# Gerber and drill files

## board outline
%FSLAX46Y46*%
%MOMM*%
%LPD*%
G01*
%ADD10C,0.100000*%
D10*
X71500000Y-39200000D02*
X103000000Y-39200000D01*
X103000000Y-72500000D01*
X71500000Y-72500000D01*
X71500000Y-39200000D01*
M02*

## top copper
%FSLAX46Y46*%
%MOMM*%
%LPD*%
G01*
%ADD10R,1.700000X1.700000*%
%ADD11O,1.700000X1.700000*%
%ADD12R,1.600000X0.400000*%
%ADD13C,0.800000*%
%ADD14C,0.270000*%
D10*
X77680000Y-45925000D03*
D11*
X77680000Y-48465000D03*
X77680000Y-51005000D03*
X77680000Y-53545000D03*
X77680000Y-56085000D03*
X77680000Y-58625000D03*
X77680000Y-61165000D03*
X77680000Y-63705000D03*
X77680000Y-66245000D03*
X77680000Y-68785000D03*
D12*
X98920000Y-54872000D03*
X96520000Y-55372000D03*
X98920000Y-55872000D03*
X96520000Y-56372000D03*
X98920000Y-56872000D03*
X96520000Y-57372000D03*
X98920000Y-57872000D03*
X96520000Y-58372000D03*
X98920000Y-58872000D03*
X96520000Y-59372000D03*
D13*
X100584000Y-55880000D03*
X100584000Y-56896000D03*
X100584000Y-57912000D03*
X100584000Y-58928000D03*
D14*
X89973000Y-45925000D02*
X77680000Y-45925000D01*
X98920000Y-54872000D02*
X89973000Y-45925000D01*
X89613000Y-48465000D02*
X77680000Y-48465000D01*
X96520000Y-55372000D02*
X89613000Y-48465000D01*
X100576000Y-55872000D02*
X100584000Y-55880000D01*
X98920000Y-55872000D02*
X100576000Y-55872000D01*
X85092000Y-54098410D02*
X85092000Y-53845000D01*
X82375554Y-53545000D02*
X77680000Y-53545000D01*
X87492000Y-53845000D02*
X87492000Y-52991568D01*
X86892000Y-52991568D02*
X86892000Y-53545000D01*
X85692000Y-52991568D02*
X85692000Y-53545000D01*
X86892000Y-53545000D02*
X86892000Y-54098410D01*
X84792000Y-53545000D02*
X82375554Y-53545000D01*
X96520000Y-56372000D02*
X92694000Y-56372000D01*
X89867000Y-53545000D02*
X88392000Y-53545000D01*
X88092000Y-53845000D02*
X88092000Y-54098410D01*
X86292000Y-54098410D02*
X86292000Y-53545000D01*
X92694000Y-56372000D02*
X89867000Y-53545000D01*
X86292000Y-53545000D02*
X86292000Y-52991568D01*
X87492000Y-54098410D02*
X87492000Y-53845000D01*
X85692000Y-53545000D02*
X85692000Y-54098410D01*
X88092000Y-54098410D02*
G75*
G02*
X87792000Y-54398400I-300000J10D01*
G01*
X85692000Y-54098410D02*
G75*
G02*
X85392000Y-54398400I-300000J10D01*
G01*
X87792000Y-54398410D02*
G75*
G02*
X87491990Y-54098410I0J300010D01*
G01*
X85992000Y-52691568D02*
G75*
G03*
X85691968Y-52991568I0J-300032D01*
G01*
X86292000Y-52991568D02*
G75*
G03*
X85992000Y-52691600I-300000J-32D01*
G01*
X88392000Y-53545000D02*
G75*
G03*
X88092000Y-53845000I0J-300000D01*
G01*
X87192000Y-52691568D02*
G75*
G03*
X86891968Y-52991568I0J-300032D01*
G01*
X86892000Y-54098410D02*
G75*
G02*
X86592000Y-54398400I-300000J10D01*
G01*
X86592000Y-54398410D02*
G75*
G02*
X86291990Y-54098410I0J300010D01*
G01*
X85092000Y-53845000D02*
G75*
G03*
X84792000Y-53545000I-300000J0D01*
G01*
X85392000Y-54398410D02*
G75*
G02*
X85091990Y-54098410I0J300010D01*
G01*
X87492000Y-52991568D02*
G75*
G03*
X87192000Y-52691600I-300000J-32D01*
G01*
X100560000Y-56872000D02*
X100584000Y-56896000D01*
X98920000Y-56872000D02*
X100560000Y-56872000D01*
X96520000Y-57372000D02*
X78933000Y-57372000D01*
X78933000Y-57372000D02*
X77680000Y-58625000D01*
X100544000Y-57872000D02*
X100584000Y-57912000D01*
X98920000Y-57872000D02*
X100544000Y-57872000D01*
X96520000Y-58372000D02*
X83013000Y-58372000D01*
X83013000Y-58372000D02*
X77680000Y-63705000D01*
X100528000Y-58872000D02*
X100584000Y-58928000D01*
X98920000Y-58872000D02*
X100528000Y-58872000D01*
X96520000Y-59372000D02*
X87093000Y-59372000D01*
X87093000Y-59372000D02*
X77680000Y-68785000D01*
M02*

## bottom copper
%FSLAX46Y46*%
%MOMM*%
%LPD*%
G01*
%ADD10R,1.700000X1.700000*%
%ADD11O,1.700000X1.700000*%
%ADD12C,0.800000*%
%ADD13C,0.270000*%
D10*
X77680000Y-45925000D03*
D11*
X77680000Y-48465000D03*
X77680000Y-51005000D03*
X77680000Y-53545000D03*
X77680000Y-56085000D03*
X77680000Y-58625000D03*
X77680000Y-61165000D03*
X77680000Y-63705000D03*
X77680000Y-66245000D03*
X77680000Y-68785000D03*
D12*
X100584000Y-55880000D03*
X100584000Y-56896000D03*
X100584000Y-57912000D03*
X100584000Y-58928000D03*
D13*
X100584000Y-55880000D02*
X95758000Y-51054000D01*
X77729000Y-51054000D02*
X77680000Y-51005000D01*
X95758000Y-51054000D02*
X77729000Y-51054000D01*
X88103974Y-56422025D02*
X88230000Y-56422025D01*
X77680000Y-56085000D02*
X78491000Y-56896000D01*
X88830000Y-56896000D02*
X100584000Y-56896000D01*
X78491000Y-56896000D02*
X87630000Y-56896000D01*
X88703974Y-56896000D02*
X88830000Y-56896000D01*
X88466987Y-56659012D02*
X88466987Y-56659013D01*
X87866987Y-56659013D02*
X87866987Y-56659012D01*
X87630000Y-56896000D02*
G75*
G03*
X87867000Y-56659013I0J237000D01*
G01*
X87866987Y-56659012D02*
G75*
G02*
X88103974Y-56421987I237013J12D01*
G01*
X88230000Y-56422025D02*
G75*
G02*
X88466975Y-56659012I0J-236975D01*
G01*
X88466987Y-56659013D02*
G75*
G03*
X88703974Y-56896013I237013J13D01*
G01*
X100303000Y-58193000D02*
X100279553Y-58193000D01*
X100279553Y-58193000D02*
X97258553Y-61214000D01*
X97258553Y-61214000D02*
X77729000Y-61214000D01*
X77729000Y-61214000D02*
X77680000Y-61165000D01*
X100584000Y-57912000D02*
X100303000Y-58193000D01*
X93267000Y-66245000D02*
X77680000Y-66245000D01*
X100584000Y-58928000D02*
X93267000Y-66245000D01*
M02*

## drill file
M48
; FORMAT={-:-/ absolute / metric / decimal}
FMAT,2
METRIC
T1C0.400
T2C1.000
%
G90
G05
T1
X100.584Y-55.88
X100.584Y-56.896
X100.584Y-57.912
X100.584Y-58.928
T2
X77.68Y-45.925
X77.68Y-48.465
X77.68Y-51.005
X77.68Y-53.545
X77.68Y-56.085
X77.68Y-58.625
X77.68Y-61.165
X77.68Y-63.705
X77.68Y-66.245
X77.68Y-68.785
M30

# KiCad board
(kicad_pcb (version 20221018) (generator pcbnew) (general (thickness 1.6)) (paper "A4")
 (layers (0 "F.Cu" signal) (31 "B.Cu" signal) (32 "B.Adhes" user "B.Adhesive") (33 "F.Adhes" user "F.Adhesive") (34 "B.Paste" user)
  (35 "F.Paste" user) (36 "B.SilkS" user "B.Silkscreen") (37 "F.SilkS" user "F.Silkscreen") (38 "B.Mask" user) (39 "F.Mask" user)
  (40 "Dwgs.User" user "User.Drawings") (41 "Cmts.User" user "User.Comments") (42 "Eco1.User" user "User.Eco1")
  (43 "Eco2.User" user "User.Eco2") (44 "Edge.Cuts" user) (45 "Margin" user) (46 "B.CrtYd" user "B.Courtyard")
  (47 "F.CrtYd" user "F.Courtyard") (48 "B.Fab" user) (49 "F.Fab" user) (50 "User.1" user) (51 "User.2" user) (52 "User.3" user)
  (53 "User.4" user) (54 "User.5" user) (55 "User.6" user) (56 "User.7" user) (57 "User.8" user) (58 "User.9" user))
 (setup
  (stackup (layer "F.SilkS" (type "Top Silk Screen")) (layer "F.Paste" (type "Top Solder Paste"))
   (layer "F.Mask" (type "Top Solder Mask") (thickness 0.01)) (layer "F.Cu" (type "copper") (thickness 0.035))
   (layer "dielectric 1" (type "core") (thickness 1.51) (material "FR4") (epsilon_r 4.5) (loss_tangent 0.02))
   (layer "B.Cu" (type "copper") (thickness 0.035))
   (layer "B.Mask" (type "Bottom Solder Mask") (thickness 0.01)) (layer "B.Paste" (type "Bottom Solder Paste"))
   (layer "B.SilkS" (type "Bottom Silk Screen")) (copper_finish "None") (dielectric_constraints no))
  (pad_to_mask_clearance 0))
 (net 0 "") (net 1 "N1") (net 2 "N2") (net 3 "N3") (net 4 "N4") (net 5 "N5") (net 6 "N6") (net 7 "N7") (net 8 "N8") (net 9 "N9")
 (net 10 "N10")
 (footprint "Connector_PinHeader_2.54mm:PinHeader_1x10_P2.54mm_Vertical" (layer "F.Cu") (at 77.68 45.925)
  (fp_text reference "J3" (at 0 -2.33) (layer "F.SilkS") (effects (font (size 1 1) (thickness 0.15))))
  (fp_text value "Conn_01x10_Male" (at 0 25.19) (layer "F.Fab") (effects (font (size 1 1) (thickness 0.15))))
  (pad "1" thru_hole rect (at 0 0) (size 1.7 1.7) (drill 1) (layers "*.Cu" "*.Mask") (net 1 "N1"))
  (pad "2" thru_hole oval (at 0 2.54) (size 1.7 1.7) (drill 1) (layers "*.Cu" "*.Mask") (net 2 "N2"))
  (pad "3" thru_hole oval (at 0 5.08) (size 1.7 1.7) (drill 1) (layers "*.Cu" "*.Mask") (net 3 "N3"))
  (pad "4" thru_hole oval (at 0 7.62) (size 1.7 1.7) (drill 1) (layers "*.Cu" "*.Mask") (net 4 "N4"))
  (pad "5" thru_hole oval (at 0 10.16) (size 1.7 1.7) (drill 1) (layers "*.Cu" "*.Mask") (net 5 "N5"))
  (pad "6" thru_hole oval (at 0 12.7) (size 1.7 1.7) (drill 1) (layers "*.Cu" "*.Mask") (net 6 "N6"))
  (pad "7" thru_hole oval (at 0 15.24) (size 1.7 1.7) (drill 1) (layers "*.Cu" "*.Mask") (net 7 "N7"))
  (pad "8" thru_hole oval (at 0 17.78) (size 1.7 1.7) (drill 1) (layers "*.Cu" "*.Mask") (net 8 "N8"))
  (pad "9" thru_hole oval (at 0 20.32) (size 1.7 1.7) (drill 1) (layers "*.Cu" "*.Mask") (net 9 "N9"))
  (pad "10" thru_hole oval (at 0 22.86) (size 1.7 1.7) (drill 1) (layers "*.Cu" "*.Mask") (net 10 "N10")))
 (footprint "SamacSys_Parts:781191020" (layer "F.Cu") (at 97.72 57.122 -90)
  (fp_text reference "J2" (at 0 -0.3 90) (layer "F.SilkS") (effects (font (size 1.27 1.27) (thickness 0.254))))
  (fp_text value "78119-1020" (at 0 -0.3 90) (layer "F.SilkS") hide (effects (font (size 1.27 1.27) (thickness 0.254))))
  (pad "1" smd rect (at -2.25 -1.2 270) (size 0.4 1.6) (layers "F.Cu" "F.Paste" "F.Mask") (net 1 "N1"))
  (pad "2" smd rect (at -1.75 1.2 270) (size 0.4 1.6) (layers "F.Cu" "F.Paste" "F.Mask") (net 2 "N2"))
  (pad "3" smd rect (at -1.25 -1.2 270) (size 0.4 1.6) (layers "F.Cu" "F.Paste" "F.Mask") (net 3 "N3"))
  (pad "4" smd rect (at -0.75 1.2 270) (size 0.4 1.6) (layers "F.Cu" "F.Paste" "F.Mask") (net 4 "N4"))
  (pad "5" smd rect (at -0.25 -1.2 270) (size 0.4 1.6) (layers "F.Cu" "F.Paste" "F.Mask") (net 5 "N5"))
  (pad "6" smd rect (at 0.25 1.2 270) (size 0.4 1.6) (layers "F.Cu" "F.Paste" "F.Mask") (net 6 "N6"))
  (pad "7" smd rect (at 0.75 -1.2 270) (size 0.4 1.6) (layers "F.Cu" "F.Paste" "F.Mask") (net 7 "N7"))
  (pad "8" smd rect (at 1.25 1.2 270) (size 0.4 1.6) (layers "F.Cu" "F.Paste" "F.Mask") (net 8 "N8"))
  (pad "9" smd rect (at 1.75 -1.2 270) (size 0.4 1.6) (layers "F.Cu" "F.Paste" "F.Mask") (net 9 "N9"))
  (pad "10" smd rect (at 2.25 1.2 270) (size 0.4 1.6) (layers "F.Cu" "F.Paste" "F.Mask") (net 10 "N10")))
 (gr_rect (start 71.5 39.2) (end 103 72.5) (stroke (width 0.1) (type solid)) (fill none) (layer "Edge.Cuts"))
 (segment (start 89.973 45.925) (end 77.68 45.925) (width 0.27) (layer "F.Cu") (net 1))
 (segment (start 98.92 54.872) (end 89.973 45.925) (width 0.27) (layer "F.Cu") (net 1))
 (segment (start 89.613 48.465) (end 77.68 48.465) (width 0.27) (layer "F.Cu") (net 2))
 (segment (start 96.52 55.372) (end 89.613 48.465) (width 0.27) (layer "F.Cu") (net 2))
 (segment (start 100.576 55.872) (end 100.584 55.88) (width 0.27) (layer "F.Cu") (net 3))
 (segment (start 98.92 55.872) (end 100.576 55.872) (width 0.27) (layer "F.Cu") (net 3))
 (via (at 100.584 55.88) (size 0.8) (drill 0.4) (layers "F.Cu" "B.Cu") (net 3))
 (segment (start 100.584 55.88) (end 95.758 51.054) (width 0.27) (layer "B.Cu") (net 3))
 (segment (start 77.729 51.054) (end 77.68 51.005) (width 0.27) (layer "B.Cu") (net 3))
 (segment (start 95.758 51.054) (end 77.729 51.054) (width 0.27) (layer "B.Cu") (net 3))
 (segment (start 85.092 54.09841) (end 85.092 53.845) (width 0.27) (layer "F.Cu") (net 4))
 (segment (start 82.375554 53.545) (end 77.68 53.545) (width 0.27) (layer "F.Cu") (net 4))
 (segment (start 87.492 53.845) (end 87.492 52.991568) (width 0.27) (layer "F.Cu") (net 4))
 (segment (start 86.892 52.991568) (end 86.892 53.545) (width 0.27) (layer "F.Cu") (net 4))
 (segment (start 85.692 52.991568) (end 85.692 53.545) (width 0.27) (layer "F.Cu") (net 4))
 (segment (start 86.892 53.545) (end 86.892 54.09841) (width 0.27) (layer "F.Cu") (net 4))
 (segment (start 84.792 53.545) (end 82.375554 53.545) (width 0.27) (layer "F.Cu") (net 4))
 (segment (start 96.52 56.372) (end 92.694 56.372) (width 0.27) (layer "F.Cu") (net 4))
 (segment (start 89.867 53.545) (end 88.392 53.545) (width 0.27) (layer "F.Cu") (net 4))
 (segment (start 88.092 53.845) (end 88.092 54.09841) (width 0.27) (layer "F.Cu") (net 4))
 (segment (start 86.292 54.09841) (end 86.292 53.545) (width 0.27) (layer "F.Cu") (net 4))
 (segment (start 92.694 56.372) (end 89.867 53.545) (width 0.27) (layer "F.Cu") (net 4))
 (segment (start 86.292 53.545) (end 86.292 52.991568) (width 0.27) (layer "F.Cu") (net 4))
 (segment (start 87.492 54.09841) (end 87.492 53.845) (width 0.27) (layer "F.Cu") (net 4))
 (segment (start 85.692 53.545) (end 85.692 54.09841) (width 0.27) (layer "F.Cu") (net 4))
 (arc (start 88.092 54.09841) (mid 88.004132 54.310542) (end 87.792 54.39841) (width 0.27) (layer "F.Cu") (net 4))
 (arc (start 85.692 54.09841) (mid 85.604132 54.310542) (end 85.392 54.39841) (width 0.27) (layer "F.Cu") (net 4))
 (arc (start 87.792 54.39841) (mid 87.579868 54.310542) (end 87.492 54.09841) (width 0.27) (layer "F.Cu") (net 4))
 (arc (start 85.992 52.691568) (mid 85.779868 52.779436) (end 85.692 52.991568) (width 0.27) (layer "F.Cu") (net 4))
 (arc (start 86.292 52.991568) (mid 86.204132 52.779436) (end 85.992 52.691568) (width 0.27) (layer "F.Cu") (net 4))
 (arc (start 88.392 53.545) (mid 88.179868 53.632868) (end 88.092 53.845) (width 0.27) (layer "F.Cu") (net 4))
 (arc (start 87.192 52.691568) (mid 86.979868 52.779436) (end 86.892 52.991568) (width 0.27) (layer "F.Cu") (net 4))
 (arc (start 86.892 54.09841) (mid 86.804132 54.310542) (end 86.592 54.39841) (width 0.27) (layer "F.Cu") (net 4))
 (arc (start 86.592 54.39841) (mid 86.379868 54.310542) (end 86.292 54.09841) (width 0.27) (layer "F.Cu") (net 4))
 (arc (start 85.092 53.845) (mid 85.004132 53.632868) (end 84.792 53.545) (width 0.27) (layer "F.Cu") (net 4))
 (arc (start 85.392 54.39841) (mid 85.179868 54.310542) (end 85.092 54.09841) (width 0.27) (layer "F.Cu") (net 4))
 (arc (start 87.492 52.991568) (mid 87.404132 52.779436) (end 87.192 52.691568) (width 0.27) (layer "F.Cu") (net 4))
 (segment (start 100.56 56.872) (end 100.584 56.896) (width 0.27) (layer "F.Cu") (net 5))
 (segment (start 98.92 56.872) (end 100.56 56.872) (width 0.27) (layer "F.Cu") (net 5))
 (via (at 100.584 56.896) (size 0.8) (drill 0.4) (layers "F.Cu" "B.Cu") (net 5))
 (segment (start 88.103974 56.422025) (end 88.23 56.422025) (width 0.27) (layer "B.Cu") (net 5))
 (segment (start 77.68 56.085) (end 78.491 56.896) (width 0.27) (layer "B.Cu") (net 5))
 (segment (start 88.83 56.896) (end 100.584 56.896) (width 0.27) (layer "B.Cu") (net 5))
 (segment (start 78.491 56.896) (end 87.63 56.896) (width 0.27) (layer "B.Cu") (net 5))
 (segment (start 88.703974 56.896) (end 88.83 56.896) (width 0.27) (layer "B.Cu") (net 5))
 (segment (start 88.466987 56.659012) (end 88.466987 56.659013) (width 0.27) (layer "B.Cu") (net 5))
 (segment (start 87.866987 56.659013) (end 87.866987 56.659012) (width 0.27) (layer "B.Cu") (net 5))
 (arc (start 87.63 56.896) (mid 87.797575 56.826588) (end 87.866987 56.659013) (width 0.27) (layer "B.Cu") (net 5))
 (arc (start 87.866987 56.659012) (mid 87.936399 56.491437) (end 88.103974 56.422025) (width 0.27) (layer "B.Cu") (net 5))
 (arc (start 88.23 56.422025) (mid 88.397575 56.491437) (end 88.466987 56.659012) (width 0.27) (layer "B.Cu") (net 5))
 (arc (start 88.466987 56.659013) (mid 88.536399 56.826588) (end 88.703974 56.896) (width 0.27) (layer "B.Cu") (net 5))
 (segment (start 96.52 57.372) (end 78.933 57.372) (width 0.27) (layer "F.Cu") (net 6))
 (segment (start 78.933 57.372) (end 77.68 58.625) (width 0.27) (layer "F.Cu") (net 6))
 (segment (start 100.544 57.872) (end 100.584 57.912) (width 0.27) (layer "F.Cu") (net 7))
 (segment (start 98.92 57.872) (end 100.544 57.872) (width 0.27) (layer "F.Cu") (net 7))
 (via (at 100.584 57.912) (size 0.8) (drill 0.4) (layers "F.Cu" "B.Cu") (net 7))
 (segment (start 100.303 58.193) (end 100.279553 58.193) (width 0.27) (layer "B.Cu") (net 7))
 (segment (start 100.279553 58.193) (end 97.258553 61.214) (width 0.27) (layer "B.Cu") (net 7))
 (segment (start 97.258553 61.214) (end 77.729 61.214) (width 0.27) (layer "B.Cu") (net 7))
 (segment (start 77.729 61.214) (end 77.68 61.165) (width 0.27) (layer "B.Cu") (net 7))
 (segment (start 100.584 57.912) (end 100.303 58.193) (width 0.27) (layer "B.Cu") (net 7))
 (segment (start 96.52 58.372) (end 83.013 58.372) (width 0.27) (layer "F.Cu") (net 8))
 (segment (start 83.013 58.372) (end 77.68 63.705) (width 0.27) (layer "F.Cu") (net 8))
 (segment (start 100.528 58.872) (end 100.584 58.928) (width 0.27) (layer "F.Cu") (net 9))
 (segment (start 98.92 58.872) (end 100.528 58.872) (width 0.27) (layer "F.Cu") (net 9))
 (via (at 100.584 58.928) (size 0.8) (drill 0.4) (layers "F.Cu" "B.Cu") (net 9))
 (segment (start 93.267 66.245) (end 77.68 66.245) (width 0.27) (layer "B.Cu") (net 9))
 (segment (start 100.584 58.928) (end 93.267 66.245) (width 0.27) (layer "B.Cu") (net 9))
 (segment (start 96.52 59.372) (end 87.093 59.372) (width 0.27) (layer "F.Cu") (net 10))
 (segment (start 87.093 59.372) (end 77.68 68.785) (width 0.27) (layer "F.Cu") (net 10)))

